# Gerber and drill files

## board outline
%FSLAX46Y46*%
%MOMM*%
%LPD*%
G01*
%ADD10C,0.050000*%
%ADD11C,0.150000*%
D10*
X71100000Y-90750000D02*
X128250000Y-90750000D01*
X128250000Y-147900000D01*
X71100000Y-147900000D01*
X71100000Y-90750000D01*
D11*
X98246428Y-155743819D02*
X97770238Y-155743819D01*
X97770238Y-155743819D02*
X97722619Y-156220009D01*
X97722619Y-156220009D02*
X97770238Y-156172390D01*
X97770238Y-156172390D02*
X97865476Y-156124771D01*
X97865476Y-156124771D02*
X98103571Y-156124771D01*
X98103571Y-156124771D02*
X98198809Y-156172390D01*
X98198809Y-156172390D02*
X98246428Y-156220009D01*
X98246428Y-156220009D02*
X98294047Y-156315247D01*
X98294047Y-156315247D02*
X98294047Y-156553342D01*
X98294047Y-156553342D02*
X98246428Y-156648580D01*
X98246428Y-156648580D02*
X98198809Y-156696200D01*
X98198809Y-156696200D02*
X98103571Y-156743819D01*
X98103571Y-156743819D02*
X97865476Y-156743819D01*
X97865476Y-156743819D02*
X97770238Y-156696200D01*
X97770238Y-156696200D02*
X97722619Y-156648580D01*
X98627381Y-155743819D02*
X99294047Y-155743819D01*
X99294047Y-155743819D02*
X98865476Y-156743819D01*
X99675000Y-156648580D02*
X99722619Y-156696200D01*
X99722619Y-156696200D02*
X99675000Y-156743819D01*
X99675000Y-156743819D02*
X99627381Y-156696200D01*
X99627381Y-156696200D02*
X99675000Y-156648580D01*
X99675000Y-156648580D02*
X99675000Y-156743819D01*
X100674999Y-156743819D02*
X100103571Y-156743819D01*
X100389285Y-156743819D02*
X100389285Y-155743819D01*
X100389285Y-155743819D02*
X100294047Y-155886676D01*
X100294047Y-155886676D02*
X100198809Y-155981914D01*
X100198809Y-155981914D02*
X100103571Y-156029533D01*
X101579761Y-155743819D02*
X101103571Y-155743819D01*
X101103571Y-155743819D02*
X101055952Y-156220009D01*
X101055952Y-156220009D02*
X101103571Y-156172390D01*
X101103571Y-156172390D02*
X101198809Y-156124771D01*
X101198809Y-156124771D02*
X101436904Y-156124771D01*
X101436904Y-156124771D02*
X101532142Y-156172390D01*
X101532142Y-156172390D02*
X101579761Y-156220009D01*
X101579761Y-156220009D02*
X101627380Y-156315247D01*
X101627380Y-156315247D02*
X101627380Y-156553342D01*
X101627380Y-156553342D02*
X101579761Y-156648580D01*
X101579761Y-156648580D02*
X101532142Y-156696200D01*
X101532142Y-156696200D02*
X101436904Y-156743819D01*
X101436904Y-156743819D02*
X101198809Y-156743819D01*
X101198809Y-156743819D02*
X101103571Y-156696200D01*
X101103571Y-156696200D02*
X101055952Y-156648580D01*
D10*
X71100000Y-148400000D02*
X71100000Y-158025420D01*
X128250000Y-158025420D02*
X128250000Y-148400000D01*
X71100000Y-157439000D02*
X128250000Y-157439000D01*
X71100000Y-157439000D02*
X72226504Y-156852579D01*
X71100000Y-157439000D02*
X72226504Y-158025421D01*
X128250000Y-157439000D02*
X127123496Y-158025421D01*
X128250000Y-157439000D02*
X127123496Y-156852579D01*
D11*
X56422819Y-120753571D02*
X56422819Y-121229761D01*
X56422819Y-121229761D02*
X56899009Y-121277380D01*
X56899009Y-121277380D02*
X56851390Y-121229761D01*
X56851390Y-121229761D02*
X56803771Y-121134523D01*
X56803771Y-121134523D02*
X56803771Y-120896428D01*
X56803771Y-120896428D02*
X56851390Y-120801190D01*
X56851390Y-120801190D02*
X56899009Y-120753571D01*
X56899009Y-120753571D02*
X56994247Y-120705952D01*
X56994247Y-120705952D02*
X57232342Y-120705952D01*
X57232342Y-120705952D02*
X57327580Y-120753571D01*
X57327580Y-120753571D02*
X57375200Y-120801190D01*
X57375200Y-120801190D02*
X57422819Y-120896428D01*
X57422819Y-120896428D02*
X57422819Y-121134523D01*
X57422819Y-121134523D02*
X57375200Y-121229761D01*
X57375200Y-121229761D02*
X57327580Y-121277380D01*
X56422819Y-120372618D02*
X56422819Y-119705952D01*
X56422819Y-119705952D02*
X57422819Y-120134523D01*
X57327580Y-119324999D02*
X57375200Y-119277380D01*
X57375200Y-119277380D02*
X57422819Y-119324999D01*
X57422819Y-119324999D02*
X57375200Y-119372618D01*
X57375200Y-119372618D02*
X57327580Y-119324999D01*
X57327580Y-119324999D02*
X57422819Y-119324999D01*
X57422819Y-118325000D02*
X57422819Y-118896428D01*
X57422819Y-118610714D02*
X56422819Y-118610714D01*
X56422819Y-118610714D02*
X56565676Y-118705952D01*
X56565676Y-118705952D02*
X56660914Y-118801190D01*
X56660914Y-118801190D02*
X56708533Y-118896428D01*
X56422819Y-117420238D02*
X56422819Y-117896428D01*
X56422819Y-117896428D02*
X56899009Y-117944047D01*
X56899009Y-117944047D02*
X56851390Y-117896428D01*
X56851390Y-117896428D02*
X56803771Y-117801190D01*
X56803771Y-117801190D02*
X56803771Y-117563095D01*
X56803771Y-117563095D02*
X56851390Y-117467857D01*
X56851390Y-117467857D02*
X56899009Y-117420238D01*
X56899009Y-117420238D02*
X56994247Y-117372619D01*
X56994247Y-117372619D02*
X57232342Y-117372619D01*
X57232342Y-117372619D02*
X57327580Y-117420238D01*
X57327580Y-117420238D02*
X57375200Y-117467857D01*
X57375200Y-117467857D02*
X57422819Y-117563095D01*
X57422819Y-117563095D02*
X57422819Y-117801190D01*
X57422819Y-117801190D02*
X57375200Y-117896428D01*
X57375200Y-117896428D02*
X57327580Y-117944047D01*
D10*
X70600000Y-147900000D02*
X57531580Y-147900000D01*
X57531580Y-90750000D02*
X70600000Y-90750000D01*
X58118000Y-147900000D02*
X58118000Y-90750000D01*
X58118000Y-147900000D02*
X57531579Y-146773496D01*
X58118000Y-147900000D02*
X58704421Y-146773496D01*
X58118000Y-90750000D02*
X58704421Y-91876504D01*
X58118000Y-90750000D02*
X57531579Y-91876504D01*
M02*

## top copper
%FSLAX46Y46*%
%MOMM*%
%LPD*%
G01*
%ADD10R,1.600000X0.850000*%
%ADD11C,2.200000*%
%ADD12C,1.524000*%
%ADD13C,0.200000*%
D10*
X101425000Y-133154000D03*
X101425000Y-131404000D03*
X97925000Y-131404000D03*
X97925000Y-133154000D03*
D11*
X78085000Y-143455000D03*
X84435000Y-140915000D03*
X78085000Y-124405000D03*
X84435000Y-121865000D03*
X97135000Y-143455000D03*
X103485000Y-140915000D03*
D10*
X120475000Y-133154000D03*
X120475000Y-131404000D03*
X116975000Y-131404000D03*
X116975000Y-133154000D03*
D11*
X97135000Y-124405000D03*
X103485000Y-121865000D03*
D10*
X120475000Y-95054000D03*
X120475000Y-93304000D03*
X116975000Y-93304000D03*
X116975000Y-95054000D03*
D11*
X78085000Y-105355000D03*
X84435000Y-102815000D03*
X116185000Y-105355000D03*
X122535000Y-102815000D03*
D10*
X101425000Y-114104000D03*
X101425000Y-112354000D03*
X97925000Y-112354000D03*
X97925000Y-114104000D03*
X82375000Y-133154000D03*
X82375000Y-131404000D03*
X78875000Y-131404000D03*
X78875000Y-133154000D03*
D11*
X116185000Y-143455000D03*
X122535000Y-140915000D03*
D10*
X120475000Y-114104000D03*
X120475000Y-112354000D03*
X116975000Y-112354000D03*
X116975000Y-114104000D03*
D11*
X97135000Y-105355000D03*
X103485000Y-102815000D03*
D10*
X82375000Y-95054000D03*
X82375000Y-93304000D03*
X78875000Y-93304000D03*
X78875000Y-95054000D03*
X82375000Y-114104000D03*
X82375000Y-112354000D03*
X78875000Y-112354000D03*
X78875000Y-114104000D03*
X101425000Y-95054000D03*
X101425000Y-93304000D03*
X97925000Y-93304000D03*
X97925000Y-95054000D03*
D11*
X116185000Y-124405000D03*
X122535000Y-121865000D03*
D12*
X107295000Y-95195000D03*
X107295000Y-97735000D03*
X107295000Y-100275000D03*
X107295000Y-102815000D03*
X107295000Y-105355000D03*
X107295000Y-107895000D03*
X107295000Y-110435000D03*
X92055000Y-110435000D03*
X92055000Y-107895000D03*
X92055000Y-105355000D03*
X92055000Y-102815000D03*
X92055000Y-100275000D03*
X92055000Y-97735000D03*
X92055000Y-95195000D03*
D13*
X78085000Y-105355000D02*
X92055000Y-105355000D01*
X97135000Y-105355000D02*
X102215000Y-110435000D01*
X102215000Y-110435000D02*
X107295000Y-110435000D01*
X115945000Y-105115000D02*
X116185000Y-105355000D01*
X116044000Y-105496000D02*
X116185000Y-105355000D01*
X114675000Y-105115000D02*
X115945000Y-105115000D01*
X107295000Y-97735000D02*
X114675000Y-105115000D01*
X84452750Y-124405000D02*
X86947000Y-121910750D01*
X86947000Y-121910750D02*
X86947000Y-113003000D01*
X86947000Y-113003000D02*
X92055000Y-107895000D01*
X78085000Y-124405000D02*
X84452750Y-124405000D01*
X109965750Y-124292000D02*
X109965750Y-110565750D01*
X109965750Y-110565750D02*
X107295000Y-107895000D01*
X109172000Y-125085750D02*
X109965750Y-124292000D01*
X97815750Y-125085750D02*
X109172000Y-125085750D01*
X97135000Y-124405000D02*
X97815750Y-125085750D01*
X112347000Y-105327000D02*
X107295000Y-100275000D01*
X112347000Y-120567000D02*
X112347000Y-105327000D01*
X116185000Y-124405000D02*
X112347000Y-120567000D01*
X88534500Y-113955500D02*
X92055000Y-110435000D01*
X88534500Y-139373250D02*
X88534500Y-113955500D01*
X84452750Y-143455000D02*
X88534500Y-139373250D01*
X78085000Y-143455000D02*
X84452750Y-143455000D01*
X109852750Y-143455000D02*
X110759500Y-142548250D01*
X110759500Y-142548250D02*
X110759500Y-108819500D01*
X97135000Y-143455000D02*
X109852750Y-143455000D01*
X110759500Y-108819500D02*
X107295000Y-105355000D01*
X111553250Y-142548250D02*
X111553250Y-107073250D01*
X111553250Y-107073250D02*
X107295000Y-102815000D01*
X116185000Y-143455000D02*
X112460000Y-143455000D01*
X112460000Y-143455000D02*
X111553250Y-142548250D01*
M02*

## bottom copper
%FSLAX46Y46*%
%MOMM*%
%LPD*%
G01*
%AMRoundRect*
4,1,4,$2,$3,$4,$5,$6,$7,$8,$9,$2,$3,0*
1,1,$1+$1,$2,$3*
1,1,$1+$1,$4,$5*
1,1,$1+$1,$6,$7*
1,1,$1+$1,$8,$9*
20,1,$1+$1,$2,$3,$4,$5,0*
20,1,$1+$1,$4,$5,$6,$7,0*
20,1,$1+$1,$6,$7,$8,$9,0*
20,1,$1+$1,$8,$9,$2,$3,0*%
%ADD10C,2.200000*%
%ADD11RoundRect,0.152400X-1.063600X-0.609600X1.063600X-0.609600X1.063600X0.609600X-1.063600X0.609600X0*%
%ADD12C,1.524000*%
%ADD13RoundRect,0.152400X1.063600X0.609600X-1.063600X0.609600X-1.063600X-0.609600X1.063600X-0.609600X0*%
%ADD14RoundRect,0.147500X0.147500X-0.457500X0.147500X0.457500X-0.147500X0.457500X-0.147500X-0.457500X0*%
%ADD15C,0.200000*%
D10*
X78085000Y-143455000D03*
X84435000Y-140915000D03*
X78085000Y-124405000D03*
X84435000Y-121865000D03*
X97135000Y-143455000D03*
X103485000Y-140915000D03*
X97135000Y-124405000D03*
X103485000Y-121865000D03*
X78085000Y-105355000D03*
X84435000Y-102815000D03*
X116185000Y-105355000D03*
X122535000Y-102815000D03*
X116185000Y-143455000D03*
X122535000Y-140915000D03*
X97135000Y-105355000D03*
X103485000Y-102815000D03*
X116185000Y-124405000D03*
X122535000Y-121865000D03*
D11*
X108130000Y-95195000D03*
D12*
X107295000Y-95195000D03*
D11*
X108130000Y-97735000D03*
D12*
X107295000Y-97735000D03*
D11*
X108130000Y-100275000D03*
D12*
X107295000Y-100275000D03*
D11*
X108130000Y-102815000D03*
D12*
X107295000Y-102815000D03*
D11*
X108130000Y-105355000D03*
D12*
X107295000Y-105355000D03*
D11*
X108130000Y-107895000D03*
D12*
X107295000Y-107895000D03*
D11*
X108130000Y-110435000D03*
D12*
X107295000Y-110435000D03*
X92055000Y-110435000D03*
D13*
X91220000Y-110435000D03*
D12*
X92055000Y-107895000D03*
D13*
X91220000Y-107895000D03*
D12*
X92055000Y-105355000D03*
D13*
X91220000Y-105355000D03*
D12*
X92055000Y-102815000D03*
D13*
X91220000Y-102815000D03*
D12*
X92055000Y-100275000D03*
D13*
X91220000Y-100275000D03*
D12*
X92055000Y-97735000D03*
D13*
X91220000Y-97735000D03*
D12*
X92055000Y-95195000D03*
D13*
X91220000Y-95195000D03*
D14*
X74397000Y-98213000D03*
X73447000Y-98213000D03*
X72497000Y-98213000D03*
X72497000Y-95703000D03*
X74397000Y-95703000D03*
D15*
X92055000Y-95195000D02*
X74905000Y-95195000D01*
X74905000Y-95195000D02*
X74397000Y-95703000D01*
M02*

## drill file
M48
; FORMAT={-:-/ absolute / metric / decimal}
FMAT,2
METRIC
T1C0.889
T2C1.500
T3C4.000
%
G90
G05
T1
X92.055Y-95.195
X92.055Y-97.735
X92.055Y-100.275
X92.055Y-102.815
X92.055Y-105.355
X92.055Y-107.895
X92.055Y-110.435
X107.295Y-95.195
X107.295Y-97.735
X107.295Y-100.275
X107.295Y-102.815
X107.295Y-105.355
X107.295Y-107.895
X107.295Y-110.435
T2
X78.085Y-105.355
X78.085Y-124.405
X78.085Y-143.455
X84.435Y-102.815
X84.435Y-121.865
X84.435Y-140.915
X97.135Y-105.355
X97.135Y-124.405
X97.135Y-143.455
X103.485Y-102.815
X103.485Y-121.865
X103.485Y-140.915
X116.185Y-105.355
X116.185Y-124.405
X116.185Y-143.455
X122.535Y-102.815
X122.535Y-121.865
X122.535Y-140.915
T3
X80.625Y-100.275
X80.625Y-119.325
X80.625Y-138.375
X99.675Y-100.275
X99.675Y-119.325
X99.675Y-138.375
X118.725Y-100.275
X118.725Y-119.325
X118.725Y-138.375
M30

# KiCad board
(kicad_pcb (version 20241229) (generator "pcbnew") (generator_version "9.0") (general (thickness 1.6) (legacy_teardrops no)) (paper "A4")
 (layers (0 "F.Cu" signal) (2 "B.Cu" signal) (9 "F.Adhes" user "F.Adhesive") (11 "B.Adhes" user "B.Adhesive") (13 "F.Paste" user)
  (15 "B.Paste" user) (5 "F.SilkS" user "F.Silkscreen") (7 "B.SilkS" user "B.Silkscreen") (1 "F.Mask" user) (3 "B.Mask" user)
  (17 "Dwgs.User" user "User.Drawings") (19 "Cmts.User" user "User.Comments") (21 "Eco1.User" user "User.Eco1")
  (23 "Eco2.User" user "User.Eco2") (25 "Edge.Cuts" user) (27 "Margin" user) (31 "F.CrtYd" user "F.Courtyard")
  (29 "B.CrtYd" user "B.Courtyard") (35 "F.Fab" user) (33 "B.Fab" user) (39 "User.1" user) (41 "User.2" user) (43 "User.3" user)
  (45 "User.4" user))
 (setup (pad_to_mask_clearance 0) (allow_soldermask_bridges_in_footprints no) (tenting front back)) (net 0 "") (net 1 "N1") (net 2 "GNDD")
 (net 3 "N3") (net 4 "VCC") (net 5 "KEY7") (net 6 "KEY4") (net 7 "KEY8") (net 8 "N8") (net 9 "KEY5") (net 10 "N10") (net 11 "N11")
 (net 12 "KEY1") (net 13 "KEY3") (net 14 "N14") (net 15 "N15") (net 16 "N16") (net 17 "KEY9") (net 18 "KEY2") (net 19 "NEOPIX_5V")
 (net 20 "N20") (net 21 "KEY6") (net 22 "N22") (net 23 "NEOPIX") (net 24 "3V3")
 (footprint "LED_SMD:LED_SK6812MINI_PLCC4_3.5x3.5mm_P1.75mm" (layer "F.Cu") (at 99.675 132.279 180)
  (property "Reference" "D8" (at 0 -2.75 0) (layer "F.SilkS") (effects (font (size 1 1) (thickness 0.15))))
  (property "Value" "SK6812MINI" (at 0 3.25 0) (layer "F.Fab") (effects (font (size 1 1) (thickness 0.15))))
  (pad "1" smd rect (at -1.75 -0.875 180) (size 1.6 0.85) (layers "F.Cu" "F.Mask" "F.Paste") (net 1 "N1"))
  (pad "2" smd rect (at -1.75 0.875 180) (size 1.6 0.85) (layers "F.Cu" "F.Mask" "F.Paste") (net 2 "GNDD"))
  (pad "3" smd rect (at 1.75 0.875 180) (size 1.6 0.85) (layers "F.Cu" "F.Mask" "F.Paste") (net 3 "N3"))
  (pad "4" smd rect (at 1.75 -0.875 180) (size 1.6 0.85) (layers "F.Cu" "F.Mask" "F.Paste") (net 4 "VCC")))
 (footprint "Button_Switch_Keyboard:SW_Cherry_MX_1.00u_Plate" (layer "F.Cu") (at 78.085 143.455 180)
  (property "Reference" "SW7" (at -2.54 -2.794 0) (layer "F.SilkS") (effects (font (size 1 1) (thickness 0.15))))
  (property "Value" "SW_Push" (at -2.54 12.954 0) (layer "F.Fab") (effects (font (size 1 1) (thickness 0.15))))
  (pad "" np_thru_hole circle (at -2.54 5.08 180) (size 4 4) (drill 4) (layers "*.Cu" "*.Mask"))
  (pad "1" thru_hole circle (at 0 0 180) (size 2.2 2.2) (drill 1.5) (layers "*.Cu" "*.Mask") (remove_unused_layers no) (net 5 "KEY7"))
  (pad "2" thru_hole circle (at -6.35 2.54 180) (size 2.2 2.2) (drill 1.5) (layers "*.Cu" "*.Mask") (remove_unused_layers no) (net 2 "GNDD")))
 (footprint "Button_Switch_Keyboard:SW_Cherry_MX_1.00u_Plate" (layer "F.Cu") (at 78.085 124.405 180)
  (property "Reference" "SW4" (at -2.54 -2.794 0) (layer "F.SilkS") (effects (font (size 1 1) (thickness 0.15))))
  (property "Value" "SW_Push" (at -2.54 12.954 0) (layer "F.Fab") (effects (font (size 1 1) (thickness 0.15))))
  (pad "" np_thru_hole circle (at -2.54 5.08 180) (size 4 4) (drill 4) (layers "*.Cu" "*.Mask"))
  (pad "1" thru_hole circle (at 0 0 180) (size 2.2 2.2) (drill 1.5) (layers "*.Cu" "*.Mask") (remove_unused_layers no) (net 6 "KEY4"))
  (pad "2" thru_hole circle (at -6.35 2.54 180) (size 2.2 2.2) (drill 1.5) (layers "*.Cu" "*.Mask") (remove_unused_layers no) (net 2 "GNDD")))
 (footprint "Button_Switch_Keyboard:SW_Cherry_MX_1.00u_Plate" (layer "F.Cu") (at 97.135 143.455 180)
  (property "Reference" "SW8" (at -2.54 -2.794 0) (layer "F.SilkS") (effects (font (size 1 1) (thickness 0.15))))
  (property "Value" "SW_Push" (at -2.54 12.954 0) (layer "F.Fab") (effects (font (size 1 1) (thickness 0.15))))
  (pad "" np_thru_hole circle (at -2.54 5.08 180) (size 4 4) (drill 4) (layers "*.Cu" "*.Mask"))
  (pad "1" thru_hole circle (at 0 0 180) (size 2.2 2.2) (drill 1.5) (layers "*.Cu" "*.Mask") (remove_unused_layers no) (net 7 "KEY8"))
  (pad "2" thru_hole circle (at -6.35 2.54 180) (size 2.2 2.2) (drill 1.5) (layers "*.Cu" "*.Mask") (remove_unused_layers no) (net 2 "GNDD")))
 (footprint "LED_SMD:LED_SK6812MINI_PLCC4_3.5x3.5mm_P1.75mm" (layer "F.Cu") (at 118.725 132.279 180)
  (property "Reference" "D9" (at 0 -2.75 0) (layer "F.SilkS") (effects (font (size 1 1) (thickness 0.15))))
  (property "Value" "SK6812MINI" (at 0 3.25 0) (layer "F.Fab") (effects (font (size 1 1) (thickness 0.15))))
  (pad "1" smd rect (at -1.75 -0.875 180) (size 1.6 0.85) (layers "F.Cu" "F.Mask" "F.Paste") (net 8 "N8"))
  (pad "2" smd rect (at -1.75 0.875 180) (size 1.6 0.85) (layers "F.Cu" "F.Mask" "F.Paste") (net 2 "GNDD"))
  (pad "3" smd rect (at 1.75 0.875 180) (size 1.6 0.85) (layers "F.Cu" "F.Mask" "F.Paste") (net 1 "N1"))
  (pad "4" smd rect (at 1.75 -0.875 180) (size 1.6 0.85) (layers "F.Cu" "F.Mask" "F.Paste") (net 4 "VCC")))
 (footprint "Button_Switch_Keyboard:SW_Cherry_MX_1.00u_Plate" (layer "F.Cu") (at 97.135 124.405 180)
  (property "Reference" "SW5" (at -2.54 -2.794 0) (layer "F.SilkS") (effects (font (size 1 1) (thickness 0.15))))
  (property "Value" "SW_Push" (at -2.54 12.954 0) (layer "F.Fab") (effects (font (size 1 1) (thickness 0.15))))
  (pad "" np_thru_hole circle (at -2.54 5.08 180) (size 4 4) (drill 4) (layers "*.Cu" "*.Mask"))
  (pad "1" thru_hole circle (at 0 0 180) (size 2.2 2.2) (drill 1.5) (layers "*.Cu" "*.Mask") (remove_unused_layers no) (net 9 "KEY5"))
  (pad "2" thru_hole circle (at -6.35 2.54 180) (size 2.2 2.2) (drill 1.5) (layers "*.Cu" "*.Mask") (remove_unused_layers no) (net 2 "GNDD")))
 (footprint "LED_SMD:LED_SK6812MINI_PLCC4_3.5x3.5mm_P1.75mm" (layer "F.Cu") (at 118.725 94.179 180)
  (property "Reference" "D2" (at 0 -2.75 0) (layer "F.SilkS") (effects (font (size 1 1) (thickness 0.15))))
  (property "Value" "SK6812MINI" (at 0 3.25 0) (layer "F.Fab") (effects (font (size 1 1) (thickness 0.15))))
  (pad "1" smd rect (at -1.75 -0.875 180) (size 1.6 0.85) (layers "F.Cu" "F.Mask" "F.Paste") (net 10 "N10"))
  (pad "2" smd rect (at -1.75 0.875 180) (size 1.6 0.85) (layers "F.Cu" "F.Mask" "F.Paste") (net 2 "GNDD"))
  (pad "3" smd rect (at 1.75 0.875 180) (size 1.6 0.85) (layers "F.Cu" "F.Mask" "F.Paste") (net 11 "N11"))
  (pad "4" smd rect (at 1.75 -0.875 180) (size 1.6 0.85) (layers "F.Cu" "F.Mask" "F.Paste") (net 4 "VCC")))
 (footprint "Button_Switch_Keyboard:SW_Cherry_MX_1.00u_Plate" (layer "F.Cu") (at 78.085 105.355 180)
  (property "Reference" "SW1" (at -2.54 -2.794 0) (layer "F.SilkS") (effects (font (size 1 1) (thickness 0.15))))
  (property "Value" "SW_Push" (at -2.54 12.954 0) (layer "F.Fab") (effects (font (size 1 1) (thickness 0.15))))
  (pad "" np_thru_hole circle (at -2.54 5.08 180) (size 4 4) (drill 4) (layers "*.Cu" "*.Mask"))
  (pad "1" thru_hole circle (at 0 0 180) (size 2.2 2.2) (drill 1.5) (layers "*.Cu" "*.Mask") (remove_unused_layers no) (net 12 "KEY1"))
  (pad "2" thru_hole circle (at -6.35 2.54 180) (size 2.2 2.2) (drill 1.5) (layers "*.Cu" "*.Mask") (remove_unused_layers no) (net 2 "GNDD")))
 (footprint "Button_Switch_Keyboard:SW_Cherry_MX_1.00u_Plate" (layer "F.Cu") (at 116.185 105.355 180)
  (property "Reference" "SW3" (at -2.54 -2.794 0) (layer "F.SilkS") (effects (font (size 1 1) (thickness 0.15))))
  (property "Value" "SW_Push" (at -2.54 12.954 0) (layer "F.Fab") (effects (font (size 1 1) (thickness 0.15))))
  (pad "" np_thru_hole circle (at -2.54 5.08 180) (size 4 4) (drill 4) (layers "*.Cu" "*.Mask"))
  (pad "1" thru_hole circle (at 0 0 180) (size 2.2 2.2) (drill 1.5) (layers "*.Cu" "*.Mask") (remove_unused_layers no) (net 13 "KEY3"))
  (pad "2" thru_hole circle (at -6.35 2.54 180) (size 2.2 2.2) (drill 1.5) (layers "*.Cu" "*.Mask") (remove_unused_layers no) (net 2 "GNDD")))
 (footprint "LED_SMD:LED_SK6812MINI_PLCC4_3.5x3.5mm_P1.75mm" (layer "F.Cu") (at 99.675 113.229 180)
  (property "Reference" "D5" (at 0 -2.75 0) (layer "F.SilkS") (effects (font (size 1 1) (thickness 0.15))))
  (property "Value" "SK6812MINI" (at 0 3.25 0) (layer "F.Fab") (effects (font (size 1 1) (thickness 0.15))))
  (pad "1" smd rect (at -1.75 -0.875 180) (size 1.6 0.85) (layers "F.Cu" "F.Mask" "F.Paste") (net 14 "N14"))
  (pad "2" smd rect (at -1.75 0.875 180) (size 1.6 0.85) (layers "F.Cu" "F.Mask" "F.Paste") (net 2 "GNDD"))
  (pad "3" smd rect (at 1.75 0.875 180) (size 1.6 0.85) (layers "F.Cu" "F.Mask" "F.Paste") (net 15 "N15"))
  (pad "4" smd rect (at 1.75 -0.875 180) (size 1.6 0.85) (layers "F.Cu" "F.Mask" "F.Paste") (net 4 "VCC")))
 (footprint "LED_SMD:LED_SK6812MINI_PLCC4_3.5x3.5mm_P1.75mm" (layer "F.Cu") (at 80.625 132.279 180)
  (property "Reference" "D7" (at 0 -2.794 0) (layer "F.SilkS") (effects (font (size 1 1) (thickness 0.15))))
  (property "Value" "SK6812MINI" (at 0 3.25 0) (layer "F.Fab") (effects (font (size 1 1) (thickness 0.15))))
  (pad "1" smd rect (at -1.75 -0.875 180) (size 1.6 0.85) (layers "F.Cu" "F.Mask" "F.Paste") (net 3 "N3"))
  (pad "2" smd rect (at -1.75 0.875 180) (size 1.6 0.85) (layers "F.Cu" "F.Mask" "F.Paste") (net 2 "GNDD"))
  (pad "3" smd rect (at 1.75 0.875 180) (size 1.6 0.85) (layers "F.Cu" "F.Mask" "F.Paste") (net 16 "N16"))
  (pad "4" smd rect (at 1.75 -0.875 180) (size 1.6 0.85) (layers "F.Cu" "F.Mask" "F.Paste") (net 4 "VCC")))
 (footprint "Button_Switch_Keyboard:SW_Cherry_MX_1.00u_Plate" (layer "F.Cu") (at 116.185 143.455 180)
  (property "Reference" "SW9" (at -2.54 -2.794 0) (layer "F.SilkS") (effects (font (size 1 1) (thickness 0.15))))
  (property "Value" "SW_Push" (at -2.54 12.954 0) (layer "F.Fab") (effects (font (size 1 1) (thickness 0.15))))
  (pad "" np_thru_hole circle (at -2.54 5.08 180) (size 4 4) (drill 4) (layers "*.Cu" "*.Mask"))
  (pad "1" thru_hole circle (at 0 0 180) (size 2.2 2.2) (drill 1.5) (layers "*.Cu" "*.Mask") (remove_unused_layers no) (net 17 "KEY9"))
  (pad "2" thru_hole circle (at -6.35 2.54 180) (size 2.2 2.2) (drill 1.5) (layers "*.Cu" "*.Mask") (remove_unused_layers no) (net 2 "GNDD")))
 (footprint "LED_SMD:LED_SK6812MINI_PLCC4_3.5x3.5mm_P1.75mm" (layer "F.Cu") (at 118.725 113.229 180)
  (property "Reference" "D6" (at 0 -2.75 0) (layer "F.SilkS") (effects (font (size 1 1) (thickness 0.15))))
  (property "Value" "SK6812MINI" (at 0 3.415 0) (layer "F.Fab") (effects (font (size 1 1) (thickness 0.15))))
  (pad "1" smd rect (at -1.75 -0.875 180) (size 1.6 0.85) (layers "F.Cu" "F.Mask" "F.Paste") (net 16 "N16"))
  (pad "2" smd rect (at -1.75 0.875 180) (size 1.6 0.85) (layers "F.Cu" "F.Mask" "F.Paste") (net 2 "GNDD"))
  (pad "3" smd rect (at 1.75 0.875 180) (size 1.6 0.85) (layers "F.Cu" "F.Mask" "F.Paste") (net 14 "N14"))
  (pad "4" smd rect (at 1.75 -0.875 180) (size 1.6 0.85) (layers "F.Cu" "F.Mask" "F.Paste") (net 4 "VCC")))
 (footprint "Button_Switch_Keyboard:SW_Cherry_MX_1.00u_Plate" (layer "F.Cu") (at 97.135 105.355 180)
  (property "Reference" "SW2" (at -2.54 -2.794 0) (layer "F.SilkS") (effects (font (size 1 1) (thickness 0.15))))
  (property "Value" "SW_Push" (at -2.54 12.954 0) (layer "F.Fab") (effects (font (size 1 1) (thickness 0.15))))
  (pad "" np_thru_hole circle (at -2.54 5.08 180) (size 4 4) (drill 4) (layers "*.Cu" "*.Mask"))
  (pad "1" thru_hole circle (at 0 0 180) (size 2.2 2.2) (drill 1.5) (layers "*.Cu" "*.Mask") (remove_unused_layers no) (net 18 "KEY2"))
  (pad "2" thru_hole circle (at -6.35 2.54 180) (size 2.2 2.2) (drill 1.5) (layers "*.Cu" "*.Mask") (remove_unused_layers no) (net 2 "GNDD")))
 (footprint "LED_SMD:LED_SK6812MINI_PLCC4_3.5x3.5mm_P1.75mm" (layer "F.Cu") (at 80.625 94.179 180)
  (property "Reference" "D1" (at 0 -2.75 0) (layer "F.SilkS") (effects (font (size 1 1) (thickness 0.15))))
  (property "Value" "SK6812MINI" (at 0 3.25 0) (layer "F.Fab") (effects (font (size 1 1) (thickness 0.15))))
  (pad "1" smd rect (at -1.75 -0.875 180) (size 1.6 0.85) (layers "F.Cu" "F.Mask" "F.Paste") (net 11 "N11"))
  (pad "2" smd rect (at -1.75 0.875 180) (size 1.6 0.85) (layers "F.Cu" "F.Mask" "F.Paste") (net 2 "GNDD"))
  (pad "3" smd rect (at 1.75 0.875 180) (size 1.6 0.85) (layers "F.Cu" "F.Mask" "F.Paste") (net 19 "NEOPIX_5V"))
  (pad "4" smd rect (at 1.75 -0.875 180) (size 1.6 0.85) (layers "F.Cu" "F.Mask" "F.Paste") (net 4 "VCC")))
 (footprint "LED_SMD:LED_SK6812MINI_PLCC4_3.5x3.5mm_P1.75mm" (layer "F.Cu") (at 80.625 113.229 180)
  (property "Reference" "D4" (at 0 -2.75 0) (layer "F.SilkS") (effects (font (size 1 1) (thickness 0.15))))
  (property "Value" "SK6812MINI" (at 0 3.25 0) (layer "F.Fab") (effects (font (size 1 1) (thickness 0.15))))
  (pad "1" smd rect (at -1.75 -0.875 180) (size 1.6 0.85) (layers "F.Cu" "F.Mask" "F.Paste") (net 15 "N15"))
  (pad "2" smd rect (at -1.75 0.875 180) (size 1.6 0.85) (layers "F.Cu" "F.Mask" "F.Paste") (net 2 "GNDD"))
  (pad "3" smd rect (at 1.75 0.875 180) (size 1.6 0.85) (layers "F.Cu" "F.Mask" "F.Paste") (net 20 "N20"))
  (pad "4" smd rect (at 1.75 -0.875 180) (size 1.6 0.85) (layers "F.Cu" "F.Mask" "F.Paste") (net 4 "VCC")))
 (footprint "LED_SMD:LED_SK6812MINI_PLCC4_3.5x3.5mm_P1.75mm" (layer "F.Cu") (at 99.675 94.179 180)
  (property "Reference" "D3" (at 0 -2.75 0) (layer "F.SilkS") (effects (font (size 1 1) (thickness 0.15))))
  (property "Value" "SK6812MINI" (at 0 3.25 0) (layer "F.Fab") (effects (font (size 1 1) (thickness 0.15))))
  (pad "1" smd rect (at -1.75 -0.875 180) (size 1.6 0.85) (layers "F.Cu" "F.Mask" "F.Paste") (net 20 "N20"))
  (pad "2" smd rect (at -1.75 0.875 180) (size 1.6 0.85) (layers "F.Cu" "F.Mask" "F.Paste") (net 2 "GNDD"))
  (pad "3" smd rect (at 1.75 0.875 180) (size 1.6 0.85) (layers "F.Cu" "F.Mask" "F.Paste") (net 10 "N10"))
  (pad "4" smd rect (at 1.75 -0.875 180) (size 1.6 0.85) (layers "F.Cu" "F.Mask" "F.Paste") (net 4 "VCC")))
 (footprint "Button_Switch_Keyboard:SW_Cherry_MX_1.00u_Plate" (layer "F.Cu") (at 116.185 124.405 180)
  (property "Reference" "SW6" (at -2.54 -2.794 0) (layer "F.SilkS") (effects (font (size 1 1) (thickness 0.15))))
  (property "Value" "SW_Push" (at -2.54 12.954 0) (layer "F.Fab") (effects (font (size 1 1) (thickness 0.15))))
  (pad "" np_thru_hole circle (at -2.54 5.08 180) (size 4 4) (drill 4) (layers "*.Cu" "*.Mask"))
  (pad "1" thru_hole circle (at 0 0 180) (size 2.2 2.2) (drill 1.5) (layers "*.Cu" "*.Mask") (remove_unused_layers no) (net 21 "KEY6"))
  (pad "2" thru_hole circle (at -6.35 2.54 180) (size 2.2 2.2) (drill 1.5) (layers "*.Cu" "*.Mask") (remove_unused_layers no) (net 2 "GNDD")))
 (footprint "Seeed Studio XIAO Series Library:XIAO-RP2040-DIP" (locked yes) (layer "B.Cu") (at 99.675 102.815 180)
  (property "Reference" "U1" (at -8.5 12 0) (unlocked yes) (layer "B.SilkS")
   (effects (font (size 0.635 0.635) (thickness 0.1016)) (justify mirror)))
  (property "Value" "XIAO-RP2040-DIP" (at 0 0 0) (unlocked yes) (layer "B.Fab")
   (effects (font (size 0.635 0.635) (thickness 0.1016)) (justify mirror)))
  (pad "1" smd roundrect (at -8.455 7.62) (size 2.432 1.524) (layers "B.Cu" "B.Mask") (roundrect_rratio 0.1) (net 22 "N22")
   (thermal_bridge_angle 45))
  (pad "1" thru_hole circle (at -7.62 7.62) (size 1.524 1.524) (drill 0.889) (layers "*.Cu" "*.Mask") (remove_unused_layers no)
   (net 22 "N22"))
  (pad "2" smd roundrect (at -8.455 5.08) (size 2.432 1.524) (layers "B.Cu" "B.Mask") (roundrect_rratio 0.1) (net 13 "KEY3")
   (thermal_bridge_angle 45))
  (pad "2" thru_hole circle (at -7.62 5.08) (size 1.524 1.524) (drill 0.889) (layers "*.Cu" "*.Mask") (remove_unused_layers no)
   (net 13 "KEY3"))
  (pad "3" smd roundrect (at -8.455 2.54) (size 2.432 1.524) (layers "B.Cu" "B.Mask") (roundrect_rratio 0.1) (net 21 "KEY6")
   (thermal_bridge_angle 45))
  (pad "3" thru_hole circle (at -7.62 2.54) (size 1.524 1.524) (drill 0.889) (layers "*.Cu" "*.Mask") (remove_unused_layers no)
   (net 21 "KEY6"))
  (pad "4" smd roundrect (at -8.455 0) (size 2.432 1.524) (layers "B.Cu" "B.Mask") (roundrect_rratio 0.1) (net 17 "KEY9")
   (thermal_bridge_angle 45))
  (pad "4" thru_hole circle (at -7.62 0) (size 1.524 1.524) (drill 0.889) (layers "*.Cu" "*.Mask") (remove_unused_layers no) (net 17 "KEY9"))
  (pad "5" smd roundrect (at -8.455 -2.54) (size 2.432 1.524) (layers "B.Cu" "B.Mask") (roundrect_rratio 0.1) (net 7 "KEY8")
   (thermal_bridge_angle 45))
  (pad "5" thru_hole circle (at -7.62 -2.54) (size 1.524 1.524) (drill 0.889) (layers "*.Cu" "*.Mask") (remove_unused_layers no)
   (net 7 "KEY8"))
  (pad "6" smd roundrect (at -8.455 -5.08) (size 2.432 1.524) (layers "B.Cu" "B.Mask") (roundrect_rratio 0.1) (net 9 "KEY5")
   (thermal_bridge_angle 45))
  (pad "6" thru_hole circle (at -7.62 -5.08) (size 1.524 1.524) (drill 0.889) (layers "*.Cu" "*.Mask") (remove_unused_layers no)
   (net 9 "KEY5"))
  (pad "7" smd roundrect (at -8.455 -7.62) (size 2.432 1.524) (layers "B.Cu" "B.Mask") (roundrect_rratio 0.1) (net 18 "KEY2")
   (thermal_bridge_angle 45))
  (pad "7" thru_hole circle (at -7.62 -7.62) (size 1.524 1.524) (drill 0.889) (layers "*.Cu" "*.Mask") (remove_unused_layers no)
   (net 18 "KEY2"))
  (pad "8" thru_hole circle (at 7.62 -7.62 180) (size 1.524 1.524) (drill 0.889) (layers "*.Cu" "*.Mask") (remove_unused_layers no)
   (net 5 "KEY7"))
  (pad "8" smd roundrect (at 8.455 -7.62 180) (size 2.432 1.524) (layers "B.Cu" "B.Mask") (roundrect_rratio 0.1) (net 5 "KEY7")
   (thermal_bridge_angle 45))
  (pad "9" thru_hole circle (at 7.62 -5.08 180) (size 1.524 1.524) (drill 0.889) (layers "*.Cu" "*.Mask") (remove_unused_layers no)
   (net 6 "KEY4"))
  (pad "9" smd roundrect (at 8.455 -5.08 180) (size 2.432 1.524) (layers "B.Cu" "B.Mask") (roundrect_rratio 0.1) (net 6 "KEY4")
   (thermal_bridge_angle 45))
  (pad "10" thru_hole circle (at 7.62 -2.54 180) (size 1.524 1.524) (drill 0.889) (layers "*.Cu" "*.Mask") (remove_unused_layers no)
   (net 12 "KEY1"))
  (pad "10" smd roundrect (at 8.455 -2.54 180) (size 2.432 1.524) (layers "B.Cu" "B.Mask") (roundrect_rratio 0.1) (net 12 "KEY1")
   (thermal_bridge_angle 45))
  (pad "11" thru_hole circle (at 7.62 0 180) (size 1.524 1.524) (drill 0.889) (layers "*.Cu" "*.Mask") (remove_unused_layers no)
   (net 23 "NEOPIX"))
  (pad "11" smd roundrect (at 8.455 0 180) (size 2.432 1.524) (layers "B.Cu" "B.Mask") (roundrect_rratio 0.1) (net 23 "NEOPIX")
   (thermal_bridge_angle 45))
  (pad "12" thru_hole circle (at 7.62 2.54 180) (size 1.524 1.524) (drill 0.889) (layers "*.Cu" "*.Mask") (remove_unused_layers no)
   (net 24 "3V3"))
  (pad "12" smd roundrect (at 8.455 2.54 180) (size 2.432 1.524) (layers "B.Cu" "B.Mask") (roundrect_rratio 0.1) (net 24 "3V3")
   (thermal_bridge_angle 45))
  (pad "13" thru_hole circle (at 7.62 5.08 180) (size 1.524 1.524) (drill 0.889) (layers "*.Cu" "*.Mask") (remove_unused_layers no)
   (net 2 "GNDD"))
  (pad "13" smd roundrect (at 8.455 5.08 180) (size 2.432 1.524) (layers "B.Cu" "B.Mask") (roundrect_rratio 0.1) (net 2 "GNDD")
   (thermal_bridge_angle 45))
  (pad "14" thru_hole circle (at 7.62 7.62 180) (size 1.524 1.524) (drill 0.889) (layers "*.Cu" "*.Mask") (remove_unused_layers no)
   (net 4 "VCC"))
  (pad "14" smd roundrect (at 8.455 7.62 180) (size 2.432 1.524) (layers "B.Cu" "B.Mask") (roundrect_rratio 0.1) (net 4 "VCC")
   (thermal_bridge_angle 45)))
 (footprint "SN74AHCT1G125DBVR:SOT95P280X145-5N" (layer "B.Cu") (at 73.447 96.958 90)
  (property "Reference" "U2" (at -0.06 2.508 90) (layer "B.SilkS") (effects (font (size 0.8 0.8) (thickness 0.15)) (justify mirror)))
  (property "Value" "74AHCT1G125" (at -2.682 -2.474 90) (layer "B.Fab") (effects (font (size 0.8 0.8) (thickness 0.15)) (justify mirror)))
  (pad "1" smd roundrect (at -1.255 0.95 90) (size 1.21 0.59) (layers "B.Cu" "B.Mask" "B.Paste") (roundrect_rratio 0.25) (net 2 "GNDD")
   (solder_mask_margin 0.102))
  (pad "2" smd roundrect (at -1.255 0 90) (size 1.21 0.59) (layers "B.Cu" "B.Mask" "B.Paste") (roundrect_rratio 0.25) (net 23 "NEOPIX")
   (solder_mask_margin 0.102))
  (pad "3" smd roundrect (at -1.255 -0.95 90) (size 1.21 0.59) (layers "B.Cu" "B.Mask" "B.Paste") (roundrect_rratio 0.25) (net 2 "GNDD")
   (solder_mask_margin 0.102))
  (pad "4" smd roundrect (at 1.255 -0.95 90) (size 1.21 0.59) (layers "B.Cu" "B.Mask" "B.Paste") (roundrect_rratio 0.25)
   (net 19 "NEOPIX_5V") (solder_mask_margin 0.102))
  (pad "5" smd roundrect (at 1.255 0.95 90) (size 1.21 0.59) (layers "B.Cu" "B.Mask" "B.Paste") (roundrect_rratio 0.25) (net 4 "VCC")
   (solder_mask_margin 0.102)))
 (gr_rect (start 71.1 90.75) (end 128.25 147.9) (stroke (width 0.05) (type default)) (fill no) (layer "Edge.Cuts"))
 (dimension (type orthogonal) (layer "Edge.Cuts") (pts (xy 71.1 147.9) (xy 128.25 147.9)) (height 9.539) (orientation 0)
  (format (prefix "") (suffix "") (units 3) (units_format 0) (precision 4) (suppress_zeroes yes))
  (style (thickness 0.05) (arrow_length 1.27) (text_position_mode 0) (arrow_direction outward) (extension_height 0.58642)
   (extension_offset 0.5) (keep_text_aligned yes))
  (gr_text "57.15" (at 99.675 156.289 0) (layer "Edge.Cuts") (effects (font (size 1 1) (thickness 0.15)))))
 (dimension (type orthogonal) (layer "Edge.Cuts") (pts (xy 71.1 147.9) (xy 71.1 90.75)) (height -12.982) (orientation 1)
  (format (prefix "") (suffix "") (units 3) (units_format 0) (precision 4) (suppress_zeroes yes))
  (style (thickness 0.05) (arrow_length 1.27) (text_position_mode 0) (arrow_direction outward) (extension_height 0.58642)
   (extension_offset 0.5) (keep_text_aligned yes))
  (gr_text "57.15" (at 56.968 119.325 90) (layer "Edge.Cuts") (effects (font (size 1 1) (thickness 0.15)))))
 (segment (start 92.055 95.195) (end 74.905 95.195) (width 0.2) (layer "B.Cu") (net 4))
 (segment (start 74.905 95.195) (end 74.397 95.703) (width 0.2) (layer "B.Cu") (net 4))
 (segment (start 78.085 105.355) (end 92.055 105.355) (width 0.2) (layer "F.Cu") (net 12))
 (segment (start 97.135 105.355) (end 102.215 110.435) (width 0.2) (layer "F.Cu") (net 18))
 (segment (start 102.215 110.435) (end 107.295 110.435) (width 0.2) (layer "F.Cu") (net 18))
 (segment (start 115.945 105.115) (end 116.185 105.355) (width 0.2) (layer "F.Cu") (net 13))
 (segment (start 116.044 105.496) (end 116.185 105.355) (width 0.2) (layer "F.Cu") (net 13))
 (segment (start 114.675 105.115) (end 115.945 105.115) (width 0.2) (layer "F.Cu") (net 13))
 (segment (start 107.295 97.735) (end 114.675 105.115) (width 0.2) (layer "F.Cu") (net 13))
 (segment (start 84.45275 124.405) (end 86.947 121.91075) (width 0.2) (layer "F.Cu") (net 6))
 (segment (start 86.947 121.91075) (end 86.947 113.003) (width 0.2) (layer "F.Cu") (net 6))
 (segment (start 86.947 113.003) (end 92.055 107.895) (width 0.2) (layer "F.Cu") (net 6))
 (segment (start 78.085 124.405) (end 84.45275 124.405) (width 0.2) (layer "F.Cu") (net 6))
 (segment (start 109.96575 124.292) (end 109.96575 110.56575) (width 0.2) (layer "F.Cu") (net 9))
 (segment (start 109.96575 110.56575) (end 107.295 107.895) (width 0.2) (layer "F.Cu") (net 9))
 (segment (start 109.172 125.08575) (end 109.96575 124.292) (width 0.2) (layer "F.Cu") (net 9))
 (segment (start 97.81575 125.08575) (end 109.172 125.08575) (width 0.2) (layer "F.Cu") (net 9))
 (segment (start 97.135 124.405) (end 97.81575 125.08575) (width 0.2) (layer "F.Cu") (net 9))
 (segment (start 112.347 105.327) (end 107.295 100.275) (width 0.2) (layer "F.Cu") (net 21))
 (segment (start 112.347 120.567) (end 112.347 105.327) (width 0.2) (layer "F.Cu") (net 21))
 (segment (start 116.185 124.405) (end 112.347 120.567) (width 0.2) (layer "F.Cu") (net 21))
 (segment (start 88.5345 113.9555) (end 92.055 110.435) (width 0.2) (layer "F.Cu") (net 5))
 (segment (start 88.5345 139.37325) (end 88.5345 113.9555) (width 0.2) (layer "F.Cu") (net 5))
 (segment (start 84.45275 143.455) (end 88.5345 139.37325) (width 0.2) (layer "F.Cu") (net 5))
 (segment (start 78.085 143.455) (end 84.45275 143.455) (width 0.2) (layer "F.Cu") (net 5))
 (segment (start 109.85275 143.455) (end 110.7595 142.54825) (width 0.2) (layer "F.Cu") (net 7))
 (segment (start 110.7595 142.54825) (end 110.7595 108.8195) (width 0.2) (layer "F.Cu") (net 7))
 (segment (start 97.135 143.455) (end 109.85275 143.455) (width 0.2) (layer "F.Cu") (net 7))
 (segment (start 110.7595 108.8195) (end 107.295 105.355) (width 0.2) (layer "F.Cu") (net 7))
 (segment (start 111.55325 142.54825) (end 111.55325 107.07325) (width 0.2) (layer "F.Cu") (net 17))
 (segment (start 111.55325 107.07325) (end 107.295 102.815) (width 0.2) (layer "F.Cu") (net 17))
 (segment (start 116.185 143.455) (end 112.46 143.455) (width 0.2) (layer "F.Cu") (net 17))
 (segment (start 112.46 143.455) (end 111.55325 142.54825) (width 0.2) (layer "F.Cu") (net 17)))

